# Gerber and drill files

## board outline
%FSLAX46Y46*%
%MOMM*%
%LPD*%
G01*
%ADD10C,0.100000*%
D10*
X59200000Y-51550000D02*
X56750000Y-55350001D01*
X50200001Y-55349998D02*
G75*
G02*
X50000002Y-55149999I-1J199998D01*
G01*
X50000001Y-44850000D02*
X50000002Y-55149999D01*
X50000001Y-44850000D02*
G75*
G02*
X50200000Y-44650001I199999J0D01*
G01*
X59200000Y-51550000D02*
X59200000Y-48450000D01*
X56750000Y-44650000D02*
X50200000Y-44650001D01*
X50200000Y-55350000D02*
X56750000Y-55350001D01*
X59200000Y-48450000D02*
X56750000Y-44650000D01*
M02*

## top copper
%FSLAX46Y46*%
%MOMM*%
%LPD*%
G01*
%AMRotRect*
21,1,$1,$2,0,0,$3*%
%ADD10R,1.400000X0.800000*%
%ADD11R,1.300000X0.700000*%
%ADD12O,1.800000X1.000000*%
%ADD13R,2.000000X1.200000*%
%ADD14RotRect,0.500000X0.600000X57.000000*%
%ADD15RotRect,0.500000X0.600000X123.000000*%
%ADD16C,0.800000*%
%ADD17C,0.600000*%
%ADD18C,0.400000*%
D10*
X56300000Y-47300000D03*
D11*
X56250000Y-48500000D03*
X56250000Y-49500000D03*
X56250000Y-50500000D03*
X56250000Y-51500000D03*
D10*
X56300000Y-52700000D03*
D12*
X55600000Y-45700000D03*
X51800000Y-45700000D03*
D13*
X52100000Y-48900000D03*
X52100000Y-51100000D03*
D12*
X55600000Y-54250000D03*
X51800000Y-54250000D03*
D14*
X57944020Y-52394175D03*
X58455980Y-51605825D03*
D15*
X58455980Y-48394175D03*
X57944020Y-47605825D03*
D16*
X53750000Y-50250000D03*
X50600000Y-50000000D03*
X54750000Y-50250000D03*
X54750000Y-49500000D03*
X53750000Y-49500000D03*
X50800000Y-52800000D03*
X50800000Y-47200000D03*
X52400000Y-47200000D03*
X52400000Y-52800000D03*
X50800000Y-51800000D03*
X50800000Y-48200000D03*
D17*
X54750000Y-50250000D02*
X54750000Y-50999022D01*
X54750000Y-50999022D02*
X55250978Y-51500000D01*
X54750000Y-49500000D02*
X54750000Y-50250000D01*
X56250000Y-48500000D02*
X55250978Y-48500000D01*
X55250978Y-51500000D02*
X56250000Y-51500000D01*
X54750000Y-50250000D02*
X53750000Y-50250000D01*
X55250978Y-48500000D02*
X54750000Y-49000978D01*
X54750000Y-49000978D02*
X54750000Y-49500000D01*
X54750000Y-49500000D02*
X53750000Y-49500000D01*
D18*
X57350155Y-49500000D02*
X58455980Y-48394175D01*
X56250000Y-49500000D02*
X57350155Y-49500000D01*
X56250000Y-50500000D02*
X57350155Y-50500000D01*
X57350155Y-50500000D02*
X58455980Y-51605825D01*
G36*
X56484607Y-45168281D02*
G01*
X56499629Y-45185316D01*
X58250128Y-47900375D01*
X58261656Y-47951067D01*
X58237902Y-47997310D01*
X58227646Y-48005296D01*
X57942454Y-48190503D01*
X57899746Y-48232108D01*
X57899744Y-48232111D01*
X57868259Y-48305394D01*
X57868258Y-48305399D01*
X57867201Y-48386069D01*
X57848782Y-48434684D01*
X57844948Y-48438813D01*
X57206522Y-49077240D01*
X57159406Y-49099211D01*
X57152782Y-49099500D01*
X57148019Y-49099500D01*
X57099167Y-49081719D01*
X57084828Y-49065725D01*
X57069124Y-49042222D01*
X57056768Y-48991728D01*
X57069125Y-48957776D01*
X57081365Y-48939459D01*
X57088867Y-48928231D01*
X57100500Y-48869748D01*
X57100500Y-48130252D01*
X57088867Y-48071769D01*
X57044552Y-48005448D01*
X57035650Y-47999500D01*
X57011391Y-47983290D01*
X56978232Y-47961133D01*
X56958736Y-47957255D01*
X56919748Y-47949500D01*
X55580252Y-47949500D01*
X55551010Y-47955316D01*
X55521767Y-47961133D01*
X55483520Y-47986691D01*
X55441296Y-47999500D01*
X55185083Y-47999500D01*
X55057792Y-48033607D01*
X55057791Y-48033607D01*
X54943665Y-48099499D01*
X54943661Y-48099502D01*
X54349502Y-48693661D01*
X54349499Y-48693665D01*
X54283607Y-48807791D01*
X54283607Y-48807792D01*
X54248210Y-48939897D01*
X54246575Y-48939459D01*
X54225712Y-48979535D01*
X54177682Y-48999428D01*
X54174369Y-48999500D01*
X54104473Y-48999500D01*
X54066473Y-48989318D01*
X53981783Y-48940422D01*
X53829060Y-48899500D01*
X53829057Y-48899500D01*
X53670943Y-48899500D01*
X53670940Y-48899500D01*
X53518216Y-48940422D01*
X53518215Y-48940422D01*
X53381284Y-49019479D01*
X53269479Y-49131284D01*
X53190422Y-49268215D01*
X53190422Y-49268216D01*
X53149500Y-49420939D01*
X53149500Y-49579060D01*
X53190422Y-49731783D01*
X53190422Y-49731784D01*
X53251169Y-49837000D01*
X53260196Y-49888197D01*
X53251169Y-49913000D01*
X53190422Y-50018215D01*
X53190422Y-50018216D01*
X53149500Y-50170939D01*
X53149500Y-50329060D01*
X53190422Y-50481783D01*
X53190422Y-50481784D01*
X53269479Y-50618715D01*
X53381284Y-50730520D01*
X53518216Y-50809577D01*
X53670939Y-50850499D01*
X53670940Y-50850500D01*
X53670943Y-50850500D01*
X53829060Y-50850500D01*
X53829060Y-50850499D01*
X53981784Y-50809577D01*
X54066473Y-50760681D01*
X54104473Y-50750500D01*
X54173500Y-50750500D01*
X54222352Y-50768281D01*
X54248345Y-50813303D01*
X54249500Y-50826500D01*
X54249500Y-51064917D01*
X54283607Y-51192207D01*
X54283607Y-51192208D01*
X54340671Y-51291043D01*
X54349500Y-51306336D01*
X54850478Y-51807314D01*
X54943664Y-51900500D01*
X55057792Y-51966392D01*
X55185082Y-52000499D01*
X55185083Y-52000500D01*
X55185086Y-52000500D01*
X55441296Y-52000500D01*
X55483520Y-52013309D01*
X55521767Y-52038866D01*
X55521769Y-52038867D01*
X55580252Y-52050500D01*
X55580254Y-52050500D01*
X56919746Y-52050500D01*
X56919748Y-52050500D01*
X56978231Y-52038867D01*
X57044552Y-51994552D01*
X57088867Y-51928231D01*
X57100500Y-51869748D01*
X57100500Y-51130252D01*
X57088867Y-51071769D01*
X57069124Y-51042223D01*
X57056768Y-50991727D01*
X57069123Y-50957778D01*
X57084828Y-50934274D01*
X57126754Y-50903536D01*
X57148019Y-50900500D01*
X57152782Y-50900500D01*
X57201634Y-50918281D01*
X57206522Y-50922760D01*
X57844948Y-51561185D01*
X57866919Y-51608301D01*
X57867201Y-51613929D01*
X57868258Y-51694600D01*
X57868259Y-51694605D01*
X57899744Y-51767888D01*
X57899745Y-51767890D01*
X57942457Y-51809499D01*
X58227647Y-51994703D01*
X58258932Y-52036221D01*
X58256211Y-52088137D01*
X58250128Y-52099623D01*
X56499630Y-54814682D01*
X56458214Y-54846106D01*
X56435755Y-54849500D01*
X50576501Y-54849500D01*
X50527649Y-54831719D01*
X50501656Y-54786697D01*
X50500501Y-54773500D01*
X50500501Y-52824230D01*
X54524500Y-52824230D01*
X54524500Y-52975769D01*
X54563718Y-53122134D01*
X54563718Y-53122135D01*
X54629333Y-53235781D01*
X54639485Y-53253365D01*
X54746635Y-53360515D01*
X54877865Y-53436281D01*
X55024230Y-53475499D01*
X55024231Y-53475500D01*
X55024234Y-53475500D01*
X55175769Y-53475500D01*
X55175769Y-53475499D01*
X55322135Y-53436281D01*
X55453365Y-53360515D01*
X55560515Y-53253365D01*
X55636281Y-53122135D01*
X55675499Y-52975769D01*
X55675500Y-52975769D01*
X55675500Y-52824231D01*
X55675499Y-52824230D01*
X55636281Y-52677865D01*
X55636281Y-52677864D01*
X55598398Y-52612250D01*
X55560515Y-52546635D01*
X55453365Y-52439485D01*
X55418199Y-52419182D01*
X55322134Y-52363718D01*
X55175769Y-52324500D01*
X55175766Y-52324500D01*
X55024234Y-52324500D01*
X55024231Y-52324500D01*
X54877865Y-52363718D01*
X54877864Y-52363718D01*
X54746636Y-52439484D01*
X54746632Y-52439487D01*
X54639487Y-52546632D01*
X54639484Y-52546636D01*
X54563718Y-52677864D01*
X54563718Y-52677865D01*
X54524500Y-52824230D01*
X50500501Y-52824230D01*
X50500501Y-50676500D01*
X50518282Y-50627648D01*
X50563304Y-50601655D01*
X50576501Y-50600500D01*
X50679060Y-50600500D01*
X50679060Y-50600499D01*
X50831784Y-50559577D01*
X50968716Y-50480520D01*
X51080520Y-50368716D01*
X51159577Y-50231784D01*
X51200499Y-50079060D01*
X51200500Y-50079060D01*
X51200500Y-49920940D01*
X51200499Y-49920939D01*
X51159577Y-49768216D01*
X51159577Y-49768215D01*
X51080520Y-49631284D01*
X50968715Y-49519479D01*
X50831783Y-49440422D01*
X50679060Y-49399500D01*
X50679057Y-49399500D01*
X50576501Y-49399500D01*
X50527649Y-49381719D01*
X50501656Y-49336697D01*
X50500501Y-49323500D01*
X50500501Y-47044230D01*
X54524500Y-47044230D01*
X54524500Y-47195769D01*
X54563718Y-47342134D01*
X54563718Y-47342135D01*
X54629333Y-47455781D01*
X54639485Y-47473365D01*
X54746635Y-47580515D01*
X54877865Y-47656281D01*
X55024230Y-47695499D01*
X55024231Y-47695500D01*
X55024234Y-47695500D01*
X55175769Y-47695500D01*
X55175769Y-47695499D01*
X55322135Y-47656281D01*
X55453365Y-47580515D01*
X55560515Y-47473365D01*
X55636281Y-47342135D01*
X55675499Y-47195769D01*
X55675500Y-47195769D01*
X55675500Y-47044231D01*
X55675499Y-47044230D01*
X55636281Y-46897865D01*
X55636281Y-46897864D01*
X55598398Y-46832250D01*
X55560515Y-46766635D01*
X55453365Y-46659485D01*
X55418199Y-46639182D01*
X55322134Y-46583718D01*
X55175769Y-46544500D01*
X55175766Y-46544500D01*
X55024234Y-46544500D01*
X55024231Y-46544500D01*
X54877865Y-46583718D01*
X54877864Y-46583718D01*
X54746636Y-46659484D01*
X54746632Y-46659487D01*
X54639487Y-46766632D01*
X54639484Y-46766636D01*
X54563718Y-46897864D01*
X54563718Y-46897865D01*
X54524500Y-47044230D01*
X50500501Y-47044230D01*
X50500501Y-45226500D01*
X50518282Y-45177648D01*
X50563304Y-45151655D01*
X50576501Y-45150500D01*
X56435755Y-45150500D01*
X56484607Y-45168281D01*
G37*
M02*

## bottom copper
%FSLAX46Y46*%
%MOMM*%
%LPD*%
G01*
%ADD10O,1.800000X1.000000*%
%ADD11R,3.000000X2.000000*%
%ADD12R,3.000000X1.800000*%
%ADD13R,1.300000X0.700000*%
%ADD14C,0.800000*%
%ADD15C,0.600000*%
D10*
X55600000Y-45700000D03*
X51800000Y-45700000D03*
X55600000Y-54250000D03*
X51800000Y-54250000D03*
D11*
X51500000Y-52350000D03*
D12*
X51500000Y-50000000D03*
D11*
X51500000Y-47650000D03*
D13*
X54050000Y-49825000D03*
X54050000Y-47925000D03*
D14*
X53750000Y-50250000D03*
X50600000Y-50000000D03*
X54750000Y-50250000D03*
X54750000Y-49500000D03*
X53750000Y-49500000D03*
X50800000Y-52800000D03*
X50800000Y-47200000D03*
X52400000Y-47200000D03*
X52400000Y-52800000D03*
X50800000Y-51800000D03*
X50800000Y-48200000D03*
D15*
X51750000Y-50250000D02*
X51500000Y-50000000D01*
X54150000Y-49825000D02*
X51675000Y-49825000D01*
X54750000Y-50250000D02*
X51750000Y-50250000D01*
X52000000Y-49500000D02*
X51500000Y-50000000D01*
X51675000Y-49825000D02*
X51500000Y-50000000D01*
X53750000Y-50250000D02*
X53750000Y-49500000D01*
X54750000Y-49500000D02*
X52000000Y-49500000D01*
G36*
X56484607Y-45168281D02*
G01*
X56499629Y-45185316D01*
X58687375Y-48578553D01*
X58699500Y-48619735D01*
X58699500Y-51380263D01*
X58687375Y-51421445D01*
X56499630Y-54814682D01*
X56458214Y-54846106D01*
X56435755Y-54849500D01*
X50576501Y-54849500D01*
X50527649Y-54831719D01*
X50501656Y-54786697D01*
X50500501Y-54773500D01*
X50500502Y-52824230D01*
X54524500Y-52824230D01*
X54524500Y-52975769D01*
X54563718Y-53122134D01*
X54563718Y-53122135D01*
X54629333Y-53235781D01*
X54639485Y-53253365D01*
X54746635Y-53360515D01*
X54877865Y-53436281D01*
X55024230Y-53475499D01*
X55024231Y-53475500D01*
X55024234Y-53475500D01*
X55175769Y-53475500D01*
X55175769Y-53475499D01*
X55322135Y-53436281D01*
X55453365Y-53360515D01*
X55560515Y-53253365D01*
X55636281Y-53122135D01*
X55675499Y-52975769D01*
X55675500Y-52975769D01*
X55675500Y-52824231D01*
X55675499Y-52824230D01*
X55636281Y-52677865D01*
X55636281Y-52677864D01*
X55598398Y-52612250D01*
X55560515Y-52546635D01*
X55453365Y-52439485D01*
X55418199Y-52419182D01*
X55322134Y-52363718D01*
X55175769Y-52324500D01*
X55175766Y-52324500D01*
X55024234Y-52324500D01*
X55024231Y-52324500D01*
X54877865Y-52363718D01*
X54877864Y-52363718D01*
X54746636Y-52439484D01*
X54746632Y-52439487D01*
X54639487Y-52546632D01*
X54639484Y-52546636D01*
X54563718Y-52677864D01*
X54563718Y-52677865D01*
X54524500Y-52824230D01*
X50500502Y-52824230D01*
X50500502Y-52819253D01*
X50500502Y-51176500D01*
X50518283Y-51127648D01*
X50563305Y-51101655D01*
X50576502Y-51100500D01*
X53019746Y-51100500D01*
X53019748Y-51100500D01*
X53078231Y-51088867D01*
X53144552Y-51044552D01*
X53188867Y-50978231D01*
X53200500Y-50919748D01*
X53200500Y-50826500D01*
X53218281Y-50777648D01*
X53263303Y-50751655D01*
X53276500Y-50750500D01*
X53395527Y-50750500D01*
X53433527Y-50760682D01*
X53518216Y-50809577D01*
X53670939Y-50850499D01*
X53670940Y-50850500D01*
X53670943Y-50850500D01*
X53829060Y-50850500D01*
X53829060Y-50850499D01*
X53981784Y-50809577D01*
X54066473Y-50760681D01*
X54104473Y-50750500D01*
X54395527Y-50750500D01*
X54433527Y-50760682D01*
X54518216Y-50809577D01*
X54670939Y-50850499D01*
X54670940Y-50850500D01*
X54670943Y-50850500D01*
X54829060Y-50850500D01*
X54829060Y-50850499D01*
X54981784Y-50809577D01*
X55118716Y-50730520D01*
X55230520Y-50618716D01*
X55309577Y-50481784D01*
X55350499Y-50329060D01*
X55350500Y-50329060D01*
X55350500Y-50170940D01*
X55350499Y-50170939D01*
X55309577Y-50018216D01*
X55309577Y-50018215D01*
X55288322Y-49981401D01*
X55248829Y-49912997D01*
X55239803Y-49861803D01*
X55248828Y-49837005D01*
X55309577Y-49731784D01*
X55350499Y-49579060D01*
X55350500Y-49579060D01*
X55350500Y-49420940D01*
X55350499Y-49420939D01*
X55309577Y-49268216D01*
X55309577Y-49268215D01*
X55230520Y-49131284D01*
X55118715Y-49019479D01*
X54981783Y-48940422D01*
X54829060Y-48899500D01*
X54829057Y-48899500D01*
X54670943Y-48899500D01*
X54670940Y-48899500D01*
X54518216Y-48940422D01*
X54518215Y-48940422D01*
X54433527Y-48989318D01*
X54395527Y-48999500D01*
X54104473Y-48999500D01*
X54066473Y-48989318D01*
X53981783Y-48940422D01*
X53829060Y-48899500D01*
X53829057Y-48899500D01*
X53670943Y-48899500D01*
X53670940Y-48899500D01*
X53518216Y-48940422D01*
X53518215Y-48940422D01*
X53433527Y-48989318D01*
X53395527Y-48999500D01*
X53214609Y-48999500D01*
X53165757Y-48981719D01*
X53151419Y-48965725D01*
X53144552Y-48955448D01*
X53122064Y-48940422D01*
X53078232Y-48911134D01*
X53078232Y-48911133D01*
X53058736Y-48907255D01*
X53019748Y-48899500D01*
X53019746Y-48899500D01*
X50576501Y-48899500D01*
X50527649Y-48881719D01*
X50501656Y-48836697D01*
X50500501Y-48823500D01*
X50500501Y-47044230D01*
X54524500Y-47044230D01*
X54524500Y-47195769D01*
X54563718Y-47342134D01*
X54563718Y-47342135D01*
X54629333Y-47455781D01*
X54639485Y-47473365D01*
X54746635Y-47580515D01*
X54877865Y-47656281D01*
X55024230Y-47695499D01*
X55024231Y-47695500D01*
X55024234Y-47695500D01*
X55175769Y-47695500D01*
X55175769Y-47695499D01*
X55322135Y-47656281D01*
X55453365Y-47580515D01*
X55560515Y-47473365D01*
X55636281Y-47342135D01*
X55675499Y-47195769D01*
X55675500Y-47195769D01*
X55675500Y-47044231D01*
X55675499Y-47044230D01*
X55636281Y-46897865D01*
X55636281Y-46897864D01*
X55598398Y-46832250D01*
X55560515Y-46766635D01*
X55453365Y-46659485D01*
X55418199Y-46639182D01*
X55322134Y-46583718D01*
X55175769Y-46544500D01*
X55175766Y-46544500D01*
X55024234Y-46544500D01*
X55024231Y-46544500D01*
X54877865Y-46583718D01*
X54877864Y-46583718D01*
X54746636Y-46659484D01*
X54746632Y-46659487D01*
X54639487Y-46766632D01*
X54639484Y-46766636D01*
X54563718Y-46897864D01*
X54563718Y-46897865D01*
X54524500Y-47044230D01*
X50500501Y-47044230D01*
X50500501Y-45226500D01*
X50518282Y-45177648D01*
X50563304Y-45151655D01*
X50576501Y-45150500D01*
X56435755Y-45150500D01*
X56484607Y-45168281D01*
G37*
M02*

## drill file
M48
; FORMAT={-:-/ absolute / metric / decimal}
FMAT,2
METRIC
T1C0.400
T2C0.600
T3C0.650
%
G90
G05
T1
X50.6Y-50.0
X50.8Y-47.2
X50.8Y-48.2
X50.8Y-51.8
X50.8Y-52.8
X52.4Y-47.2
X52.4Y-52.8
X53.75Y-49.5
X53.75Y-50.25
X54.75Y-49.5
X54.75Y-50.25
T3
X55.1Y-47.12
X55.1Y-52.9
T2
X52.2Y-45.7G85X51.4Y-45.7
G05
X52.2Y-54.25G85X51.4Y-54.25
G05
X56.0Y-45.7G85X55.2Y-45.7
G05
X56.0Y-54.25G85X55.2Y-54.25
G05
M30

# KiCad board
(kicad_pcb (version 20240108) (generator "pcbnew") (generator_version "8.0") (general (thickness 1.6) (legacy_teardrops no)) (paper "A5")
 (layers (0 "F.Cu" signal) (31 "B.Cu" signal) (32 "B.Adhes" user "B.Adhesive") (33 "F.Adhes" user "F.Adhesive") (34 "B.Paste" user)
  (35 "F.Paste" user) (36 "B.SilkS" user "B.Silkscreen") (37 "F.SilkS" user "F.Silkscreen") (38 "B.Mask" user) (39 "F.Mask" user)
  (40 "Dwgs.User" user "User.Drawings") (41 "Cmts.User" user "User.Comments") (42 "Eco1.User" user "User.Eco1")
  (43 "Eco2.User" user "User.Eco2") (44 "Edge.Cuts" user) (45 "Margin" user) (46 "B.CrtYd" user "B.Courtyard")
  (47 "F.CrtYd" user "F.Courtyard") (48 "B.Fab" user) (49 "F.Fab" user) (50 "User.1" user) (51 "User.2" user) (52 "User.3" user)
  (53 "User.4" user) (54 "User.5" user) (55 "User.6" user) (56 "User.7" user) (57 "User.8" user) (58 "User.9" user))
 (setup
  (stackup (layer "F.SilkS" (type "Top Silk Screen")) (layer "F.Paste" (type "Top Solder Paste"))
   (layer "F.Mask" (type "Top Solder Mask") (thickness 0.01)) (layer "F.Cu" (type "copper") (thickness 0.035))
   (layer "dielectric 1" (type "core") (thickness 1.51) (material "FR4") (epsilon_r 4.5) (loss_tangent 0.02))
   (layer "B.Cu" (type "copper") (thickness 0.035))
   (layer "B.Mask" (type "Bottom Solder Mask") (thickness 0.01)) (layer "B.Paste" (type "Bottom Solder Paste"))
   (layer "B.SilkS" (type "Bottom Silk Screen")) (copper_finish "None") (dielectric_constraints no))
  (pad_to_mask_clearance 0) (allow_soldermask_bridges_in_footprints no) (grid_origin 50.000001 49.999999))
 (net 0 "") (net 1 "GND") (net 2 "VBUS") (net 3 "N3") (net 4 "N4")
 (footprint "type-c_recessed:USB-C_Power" (layer "F.Cu") (at 55.6 50 -90)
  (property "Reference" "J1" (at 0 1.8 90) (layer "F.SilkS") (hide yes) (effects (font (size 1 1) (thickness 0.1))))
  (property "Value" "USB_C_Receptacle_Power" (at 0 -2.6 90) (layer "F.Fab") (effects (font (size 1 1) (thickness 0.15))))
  (pad "" np_thru_hole circle (at -2.88 0.5 270) (size 0.65 0.65) (drill 0.65) (layers "*.Cu" "*.Mask"))
  (pad "" np_thru_hole circle (at 2.9 0.5 270) (size 0.65 0.65) (drill 0.65) (layers "*.Cu" "*.Mask"))
  (pad "1" smd rect (at -2.7 -0.7 270) (size 0.8 1.4) (layers "F.Cu" "F.Paste" "F.Mask") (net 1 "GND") (solder_paste_margin_ratio -0.1))
  (pad "2" smd rect (at -1.5 -0.65 270) (size 0.7 1.3) (layers "F.Cu" "F.Paste" "F.Mask") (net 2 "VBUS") (solder_paste_margin_ratio -0.07))
  (pad "3" smd rect (at -0.5 -0.65 270) (size 0.7 1.3) (layers "F.Cu" "F.Paste" "F.Mask") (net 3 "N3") (solder_paste_margin_ratio -0.07))
  (pad "4" smd rect (at 0.5 -0.65 270) (size 0.7 1.3) (layers "F.Cu" "F.Paste" "F.Mask") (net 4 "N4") (solder_paste_margin_ratio -0.07))
  (pad "5" smd rect (at 1.5 -0.65 270) (size 0.7 1.3) (layers "F.Cu" "F.Paste" "F.Mask") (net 2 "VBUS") (solder_paste_margin_ratio -0.07))
  (pad "6" smd rect (at 2.7 -0.7 270) (size 0.8 1.4) (layers "F.Cu" "F.Paste" "F.Mask") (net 1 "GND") (solder_paste_margin_ratio -0.1))
  (pad "S1" thru_hole oval (at -4.3 0 270) (size 1 1.8) (drill oval 0.6 1.4) (layers "*.Cu" "*.Mask" "F.Paste") (remove_unused_layers no)
   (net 1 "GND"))
  (pad "S1" thru_hole oval (at -4.3 3.8 270) (size 1 1.8) (drill oval 0.6 1.4) (layers "*.Cu" "*.Mask" "F.Paste") (remove_unused_layers no)
   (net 1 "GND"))
  (pad "S1" smd rect (at -1.1 3.5 270) (size 1.2 2) (layers "F.Cu" "F.Paste" "F.Mask") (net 1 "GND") (solder_paste_margin_ratio -0.2))
  (pad "S1" smd rect (at 1.1 3.5 90) (size 1.2 2) (layers "F.Cu" "F.Paste" "F.Mask") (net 1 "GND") (solder_paste_margin_ratio -0.2))
  (pad "S1" thru_hole oval (at 4.25 0 270) (size 1 1.8) (drill oval 0.6 1.4) (layers "*.Cu" "*.Mask" "F.Paste") (remove_unused_layers no)
   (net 1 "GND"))
  (pad "S1" thru_hole oval (at 4.25 3.8 270) (size 1 1.8) (drill oval 0.6 1.4) (layers "*.Cu" "*.Mask" "F.Paste") (remove_unused_layers no)
   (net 1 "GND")))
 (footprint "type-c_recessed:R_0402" (layer "F.Cu") (at 58.2 52 57)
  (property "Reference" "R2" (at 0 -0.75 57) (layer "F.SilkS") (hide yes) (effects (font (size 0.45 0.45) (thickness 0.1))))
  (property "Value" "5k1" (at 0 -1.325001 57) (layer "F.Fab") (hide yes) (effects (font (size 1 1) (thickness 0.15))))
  (pad "1" smd rect (at -0.47 0 57) (size 0.5 0.6) (layers "F.Cu" "F.Paste" "F.Mask") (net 1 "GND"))
  (pad "2" smd rect (at 0.47 0 57) (size 0.5 0.6) (layers "F.Cu" "F.Paste" "F.Mask") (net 4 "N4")))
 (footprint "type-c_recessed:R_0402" (layer "F.Cu") (at 58.2 48 123)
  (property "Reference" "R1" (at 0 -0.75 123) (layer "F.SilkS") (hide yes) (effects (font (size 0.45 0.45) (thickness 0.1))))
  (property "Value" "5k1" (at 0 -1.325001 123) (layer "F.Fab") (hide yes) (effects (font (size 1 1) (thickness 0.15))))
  (pad "1" smd rect (at -0.47 0 123) (size 0.5 0.6) (layers "F.Cu" "F.Paste" "F.Mask") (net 3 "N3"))
  (pad "2" smd rect (at 0.47 0 123) (size 0.5 0.6) (layers "F.Cu" "F.Paste" "F.Mask") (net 1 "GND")))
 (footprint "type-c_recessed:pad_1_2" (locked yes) (layer "B.Cu") (at 51.5 52.35 -90)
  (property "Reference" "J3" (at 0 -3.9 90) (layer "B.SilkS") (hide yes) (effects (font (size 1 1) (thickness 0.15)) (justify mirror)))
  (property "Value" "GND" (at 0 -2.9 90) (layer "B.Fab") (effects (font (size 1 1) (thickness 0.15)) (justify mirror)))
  (pad "1" smd rect (at 0 0 270) (size 2 3) (layers "B.Cu" "B.Paste" "B.Mask") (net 1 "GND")))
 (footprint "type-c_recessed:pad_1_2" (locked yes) (layer "B.Cu") (at 51.5 50 -90)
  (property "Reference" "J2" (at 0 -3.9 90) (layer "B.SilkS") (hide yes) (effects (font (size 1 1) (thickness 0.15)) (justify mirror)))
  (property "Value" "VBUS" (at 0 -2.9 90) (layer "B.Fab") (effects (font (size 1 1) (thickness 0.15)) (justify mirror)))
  (pad "1" smd rect (at 0 0 270) (size 1.8 3) (layers "B.Cu" "B.Paste" "B.Mask") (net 2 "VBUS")))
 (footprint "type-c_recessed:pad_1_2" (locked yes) (layer "B.Cu") (at 51.5 47.65 -90)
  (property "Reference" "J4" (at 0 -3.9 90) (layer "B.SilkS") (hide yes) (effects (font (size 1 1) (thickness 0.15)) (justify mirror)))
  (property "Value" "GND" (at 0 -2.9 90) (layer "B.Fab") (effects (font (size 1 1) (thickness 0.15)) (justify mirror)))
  (pad "1" smd rect (at 0 0 270) (size 2 3) (layers "B.Cu" "B.Paste" "B.Mask") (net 1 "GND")))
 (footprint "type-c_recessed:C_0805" (layer "B.Cu") (at 54.05 48.875 90)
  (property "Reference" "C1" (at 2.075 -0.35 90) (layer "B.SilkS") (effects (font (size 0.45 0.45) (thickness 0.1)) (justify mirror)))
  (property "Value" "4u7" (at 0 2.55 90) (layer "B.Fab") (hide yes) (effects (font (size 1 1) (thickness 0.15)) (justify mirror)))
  (pad "1" smd rect (at -0.95 0 90) (size 0.7 1.3) (layers "B.Cu" "B.Paste" "B.Mask") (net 2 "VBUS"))
  (pad "2" smd rect (at 0.95 0 90) (size 0.7 1.3) (layers "B.Cu" "B.Paste" "B.Mask") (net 1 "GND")))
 (gr_line (start 59.2 51.55) (end 56.75 55.350001) (stroke (width 0.1) (type solid)) (layer "Edge.Cuts"))
 (gr_arc (start 50.200001 55.349998) (mid 50.05858 55.29142) (end 50.000002 55.149999) (stroke (width 0.1) (type solid)) (layer "Edge.Cuts"))
 (gr_line (start 50.000001 44.85) (end 50.000002 55.149999) (stroke (width 0.1) (type solid)) (layer "Edge.Cuts"))
 (gr_arc (start 50.000001 44.85) (mid 50.058579 44.708579) (end 50.2 44.650001) (stroke (width 0.1) (type solid)) (layer "Edge.Cuts"))
 (gr_line (start 59.2 51.55) (end 59.2 48.45) (stroke (width 0.1) (type solid)) (layer "Edge.Cuts"))
 (gr_line (start 56.75 44.65) (end 50.2 44.650001) (stroke (width 0.1) (type solid)) (layer "Edge.Cuts"))
 (gr_line (start 50.2 55.35) (end 56.75 55.350001) (stroke (width 0.1) (type solid)) (layer "Edge.Cuts"))
 (gr_line (start 59.2 48.45) (end 56.75 44.65) (stroke (width 0.1) (type solid)) (layer "Edge.Cuts"))
 (segment (start 54.75 50.25) (end 54.75 50.999022) (width 0.6) (layer "F.Cu") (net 2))
 (segment (start 54.75 50.999022) (end 55.250978 51.5) (width 0.6) (layer "F.Cu") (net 2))
 (segment (start 54.75 49.5) (end 54.75 50.25) (width 0.6) (layer "F.Cu") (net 2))
 (segment (start 56.25 48.5) (end 55.250978 48.5) (width 0.6) (layer "F.Cu") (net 2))
 (segment (start 55.250978 51.5) (end 56.25 51.5) (width 0.6) (layer "F.Cu") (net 2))
 (segment (start 54.75 50.25) (end 53.75 50.25) (width 0.6) (layer "F.Cu") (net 2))
 (segment (start 55.250978 48.5) (end 54.75 49.000978) (width 0.6) (layer "F.Cu") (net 2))
 (segment (start 54.75 49.000978) (end 54.75 49.5) (width 0.6) (layer "F.Cu") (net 2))
 (segment (start 54.75 49.5) (end 53.75 49.5) (width 0.6) (layer "F.Cu") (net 2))
 (via (at 53.75 50.25) (size 0.8) (drill 0.4) (layers "F.Cu" "B.Cu") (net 2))
 (via (at 50.6 50) (size 0.8) (drill 0.4) (layers "F.Cu" "B.Cu") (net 2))
 (via (at 54.75 50.25) (size 0.8) (drill 0.4) (layers "F.Cu" "B.Cu") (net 2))
 (via (at 54.75 49.5) (size 0.8) (drill 0.4) (layers "F.Cu" "B.Cu") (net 2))
 (via (at 53.75 49.5) (size 0.8) (drill 0.4) (layers "F.Cu" "B.Cu") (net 2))
 (segment (start 51.75 50.25) (end 51.5 50) (width 0.6) (layer "B.Cu") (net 2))
 (segment (start 54.15 49.825) (end 51.675 49.825) (width 0.6) (layer "B.Cu") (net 2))
 (segment (start 54.75 50.25) (end 51.75 50.25) (width 0.6) (layer "B.Cu") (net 2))
 (segment (start 52 49.5) (end 51.5 50) (width 0.6) (layer "B.Cu") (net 2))
 (segment (start 51.675 49.825) (end 51.5 50) (width 0.6) (layer "B.Cu") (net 2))
 (segment (start 53.75 50.25) (end 53.75 49.5) (width 0.6) (layer "B.Cu") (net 2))
 (segment (start 54.75 49.5) (end 52 49.5) (width 0.6) (layer "B.Cu") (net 2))
 (via (at 50.8 52.8) (size 0.8) (drill 0.4) (layers "F.Cu" "B.Cu") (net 1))
 (via (at 50.8 47.2) (size 0.8) (drill 0.4) (layers "F.Cu" "B.Cu") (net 1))
 (via (at 52.4 47.2) (size 0.8) (drill 0.4) (layers "F.Cu" "B.Cu") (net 1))
 (via (at 52.4 52.8) (size 0.8) (drill 0.4) (layers "F.Cu" "B.Cu") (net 1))
 (via (at 50.8 51.8) (size 0.8) (drill 0.4) (layers "F.Cu" "B.Cu") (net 1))
 (via (at 50.8 48.2) (size 0.8) (drill 0.4) (layers "F.Cu" "B.Cu") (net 1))
 (segment (start 57.350155 49.5) (end 58.45598 48.394175) (width 0.4) (layer "F.Cu") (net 3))
 (segment (start 56.25 49.5) (end 57.350155 49.5) (width 0.4) (layer "F.Cu") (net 3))
 (segment (start 56.25 50.5) (end 57.350155 50.5) (width 0.4) (layer "F.Cu") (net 4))
 (segment (start 57.350155 50.5) (end 58.45598 51.605825) (width 0.4) (layer "F.Cu") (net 4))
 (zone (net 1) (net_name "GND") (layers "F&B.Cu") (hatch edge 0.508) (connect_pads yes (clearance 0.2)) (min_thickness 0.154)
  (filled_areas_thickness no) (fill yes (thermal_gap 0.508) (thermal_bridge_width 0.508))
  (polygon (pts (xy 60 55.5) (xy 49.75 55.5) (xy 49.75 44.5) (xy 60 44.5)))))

